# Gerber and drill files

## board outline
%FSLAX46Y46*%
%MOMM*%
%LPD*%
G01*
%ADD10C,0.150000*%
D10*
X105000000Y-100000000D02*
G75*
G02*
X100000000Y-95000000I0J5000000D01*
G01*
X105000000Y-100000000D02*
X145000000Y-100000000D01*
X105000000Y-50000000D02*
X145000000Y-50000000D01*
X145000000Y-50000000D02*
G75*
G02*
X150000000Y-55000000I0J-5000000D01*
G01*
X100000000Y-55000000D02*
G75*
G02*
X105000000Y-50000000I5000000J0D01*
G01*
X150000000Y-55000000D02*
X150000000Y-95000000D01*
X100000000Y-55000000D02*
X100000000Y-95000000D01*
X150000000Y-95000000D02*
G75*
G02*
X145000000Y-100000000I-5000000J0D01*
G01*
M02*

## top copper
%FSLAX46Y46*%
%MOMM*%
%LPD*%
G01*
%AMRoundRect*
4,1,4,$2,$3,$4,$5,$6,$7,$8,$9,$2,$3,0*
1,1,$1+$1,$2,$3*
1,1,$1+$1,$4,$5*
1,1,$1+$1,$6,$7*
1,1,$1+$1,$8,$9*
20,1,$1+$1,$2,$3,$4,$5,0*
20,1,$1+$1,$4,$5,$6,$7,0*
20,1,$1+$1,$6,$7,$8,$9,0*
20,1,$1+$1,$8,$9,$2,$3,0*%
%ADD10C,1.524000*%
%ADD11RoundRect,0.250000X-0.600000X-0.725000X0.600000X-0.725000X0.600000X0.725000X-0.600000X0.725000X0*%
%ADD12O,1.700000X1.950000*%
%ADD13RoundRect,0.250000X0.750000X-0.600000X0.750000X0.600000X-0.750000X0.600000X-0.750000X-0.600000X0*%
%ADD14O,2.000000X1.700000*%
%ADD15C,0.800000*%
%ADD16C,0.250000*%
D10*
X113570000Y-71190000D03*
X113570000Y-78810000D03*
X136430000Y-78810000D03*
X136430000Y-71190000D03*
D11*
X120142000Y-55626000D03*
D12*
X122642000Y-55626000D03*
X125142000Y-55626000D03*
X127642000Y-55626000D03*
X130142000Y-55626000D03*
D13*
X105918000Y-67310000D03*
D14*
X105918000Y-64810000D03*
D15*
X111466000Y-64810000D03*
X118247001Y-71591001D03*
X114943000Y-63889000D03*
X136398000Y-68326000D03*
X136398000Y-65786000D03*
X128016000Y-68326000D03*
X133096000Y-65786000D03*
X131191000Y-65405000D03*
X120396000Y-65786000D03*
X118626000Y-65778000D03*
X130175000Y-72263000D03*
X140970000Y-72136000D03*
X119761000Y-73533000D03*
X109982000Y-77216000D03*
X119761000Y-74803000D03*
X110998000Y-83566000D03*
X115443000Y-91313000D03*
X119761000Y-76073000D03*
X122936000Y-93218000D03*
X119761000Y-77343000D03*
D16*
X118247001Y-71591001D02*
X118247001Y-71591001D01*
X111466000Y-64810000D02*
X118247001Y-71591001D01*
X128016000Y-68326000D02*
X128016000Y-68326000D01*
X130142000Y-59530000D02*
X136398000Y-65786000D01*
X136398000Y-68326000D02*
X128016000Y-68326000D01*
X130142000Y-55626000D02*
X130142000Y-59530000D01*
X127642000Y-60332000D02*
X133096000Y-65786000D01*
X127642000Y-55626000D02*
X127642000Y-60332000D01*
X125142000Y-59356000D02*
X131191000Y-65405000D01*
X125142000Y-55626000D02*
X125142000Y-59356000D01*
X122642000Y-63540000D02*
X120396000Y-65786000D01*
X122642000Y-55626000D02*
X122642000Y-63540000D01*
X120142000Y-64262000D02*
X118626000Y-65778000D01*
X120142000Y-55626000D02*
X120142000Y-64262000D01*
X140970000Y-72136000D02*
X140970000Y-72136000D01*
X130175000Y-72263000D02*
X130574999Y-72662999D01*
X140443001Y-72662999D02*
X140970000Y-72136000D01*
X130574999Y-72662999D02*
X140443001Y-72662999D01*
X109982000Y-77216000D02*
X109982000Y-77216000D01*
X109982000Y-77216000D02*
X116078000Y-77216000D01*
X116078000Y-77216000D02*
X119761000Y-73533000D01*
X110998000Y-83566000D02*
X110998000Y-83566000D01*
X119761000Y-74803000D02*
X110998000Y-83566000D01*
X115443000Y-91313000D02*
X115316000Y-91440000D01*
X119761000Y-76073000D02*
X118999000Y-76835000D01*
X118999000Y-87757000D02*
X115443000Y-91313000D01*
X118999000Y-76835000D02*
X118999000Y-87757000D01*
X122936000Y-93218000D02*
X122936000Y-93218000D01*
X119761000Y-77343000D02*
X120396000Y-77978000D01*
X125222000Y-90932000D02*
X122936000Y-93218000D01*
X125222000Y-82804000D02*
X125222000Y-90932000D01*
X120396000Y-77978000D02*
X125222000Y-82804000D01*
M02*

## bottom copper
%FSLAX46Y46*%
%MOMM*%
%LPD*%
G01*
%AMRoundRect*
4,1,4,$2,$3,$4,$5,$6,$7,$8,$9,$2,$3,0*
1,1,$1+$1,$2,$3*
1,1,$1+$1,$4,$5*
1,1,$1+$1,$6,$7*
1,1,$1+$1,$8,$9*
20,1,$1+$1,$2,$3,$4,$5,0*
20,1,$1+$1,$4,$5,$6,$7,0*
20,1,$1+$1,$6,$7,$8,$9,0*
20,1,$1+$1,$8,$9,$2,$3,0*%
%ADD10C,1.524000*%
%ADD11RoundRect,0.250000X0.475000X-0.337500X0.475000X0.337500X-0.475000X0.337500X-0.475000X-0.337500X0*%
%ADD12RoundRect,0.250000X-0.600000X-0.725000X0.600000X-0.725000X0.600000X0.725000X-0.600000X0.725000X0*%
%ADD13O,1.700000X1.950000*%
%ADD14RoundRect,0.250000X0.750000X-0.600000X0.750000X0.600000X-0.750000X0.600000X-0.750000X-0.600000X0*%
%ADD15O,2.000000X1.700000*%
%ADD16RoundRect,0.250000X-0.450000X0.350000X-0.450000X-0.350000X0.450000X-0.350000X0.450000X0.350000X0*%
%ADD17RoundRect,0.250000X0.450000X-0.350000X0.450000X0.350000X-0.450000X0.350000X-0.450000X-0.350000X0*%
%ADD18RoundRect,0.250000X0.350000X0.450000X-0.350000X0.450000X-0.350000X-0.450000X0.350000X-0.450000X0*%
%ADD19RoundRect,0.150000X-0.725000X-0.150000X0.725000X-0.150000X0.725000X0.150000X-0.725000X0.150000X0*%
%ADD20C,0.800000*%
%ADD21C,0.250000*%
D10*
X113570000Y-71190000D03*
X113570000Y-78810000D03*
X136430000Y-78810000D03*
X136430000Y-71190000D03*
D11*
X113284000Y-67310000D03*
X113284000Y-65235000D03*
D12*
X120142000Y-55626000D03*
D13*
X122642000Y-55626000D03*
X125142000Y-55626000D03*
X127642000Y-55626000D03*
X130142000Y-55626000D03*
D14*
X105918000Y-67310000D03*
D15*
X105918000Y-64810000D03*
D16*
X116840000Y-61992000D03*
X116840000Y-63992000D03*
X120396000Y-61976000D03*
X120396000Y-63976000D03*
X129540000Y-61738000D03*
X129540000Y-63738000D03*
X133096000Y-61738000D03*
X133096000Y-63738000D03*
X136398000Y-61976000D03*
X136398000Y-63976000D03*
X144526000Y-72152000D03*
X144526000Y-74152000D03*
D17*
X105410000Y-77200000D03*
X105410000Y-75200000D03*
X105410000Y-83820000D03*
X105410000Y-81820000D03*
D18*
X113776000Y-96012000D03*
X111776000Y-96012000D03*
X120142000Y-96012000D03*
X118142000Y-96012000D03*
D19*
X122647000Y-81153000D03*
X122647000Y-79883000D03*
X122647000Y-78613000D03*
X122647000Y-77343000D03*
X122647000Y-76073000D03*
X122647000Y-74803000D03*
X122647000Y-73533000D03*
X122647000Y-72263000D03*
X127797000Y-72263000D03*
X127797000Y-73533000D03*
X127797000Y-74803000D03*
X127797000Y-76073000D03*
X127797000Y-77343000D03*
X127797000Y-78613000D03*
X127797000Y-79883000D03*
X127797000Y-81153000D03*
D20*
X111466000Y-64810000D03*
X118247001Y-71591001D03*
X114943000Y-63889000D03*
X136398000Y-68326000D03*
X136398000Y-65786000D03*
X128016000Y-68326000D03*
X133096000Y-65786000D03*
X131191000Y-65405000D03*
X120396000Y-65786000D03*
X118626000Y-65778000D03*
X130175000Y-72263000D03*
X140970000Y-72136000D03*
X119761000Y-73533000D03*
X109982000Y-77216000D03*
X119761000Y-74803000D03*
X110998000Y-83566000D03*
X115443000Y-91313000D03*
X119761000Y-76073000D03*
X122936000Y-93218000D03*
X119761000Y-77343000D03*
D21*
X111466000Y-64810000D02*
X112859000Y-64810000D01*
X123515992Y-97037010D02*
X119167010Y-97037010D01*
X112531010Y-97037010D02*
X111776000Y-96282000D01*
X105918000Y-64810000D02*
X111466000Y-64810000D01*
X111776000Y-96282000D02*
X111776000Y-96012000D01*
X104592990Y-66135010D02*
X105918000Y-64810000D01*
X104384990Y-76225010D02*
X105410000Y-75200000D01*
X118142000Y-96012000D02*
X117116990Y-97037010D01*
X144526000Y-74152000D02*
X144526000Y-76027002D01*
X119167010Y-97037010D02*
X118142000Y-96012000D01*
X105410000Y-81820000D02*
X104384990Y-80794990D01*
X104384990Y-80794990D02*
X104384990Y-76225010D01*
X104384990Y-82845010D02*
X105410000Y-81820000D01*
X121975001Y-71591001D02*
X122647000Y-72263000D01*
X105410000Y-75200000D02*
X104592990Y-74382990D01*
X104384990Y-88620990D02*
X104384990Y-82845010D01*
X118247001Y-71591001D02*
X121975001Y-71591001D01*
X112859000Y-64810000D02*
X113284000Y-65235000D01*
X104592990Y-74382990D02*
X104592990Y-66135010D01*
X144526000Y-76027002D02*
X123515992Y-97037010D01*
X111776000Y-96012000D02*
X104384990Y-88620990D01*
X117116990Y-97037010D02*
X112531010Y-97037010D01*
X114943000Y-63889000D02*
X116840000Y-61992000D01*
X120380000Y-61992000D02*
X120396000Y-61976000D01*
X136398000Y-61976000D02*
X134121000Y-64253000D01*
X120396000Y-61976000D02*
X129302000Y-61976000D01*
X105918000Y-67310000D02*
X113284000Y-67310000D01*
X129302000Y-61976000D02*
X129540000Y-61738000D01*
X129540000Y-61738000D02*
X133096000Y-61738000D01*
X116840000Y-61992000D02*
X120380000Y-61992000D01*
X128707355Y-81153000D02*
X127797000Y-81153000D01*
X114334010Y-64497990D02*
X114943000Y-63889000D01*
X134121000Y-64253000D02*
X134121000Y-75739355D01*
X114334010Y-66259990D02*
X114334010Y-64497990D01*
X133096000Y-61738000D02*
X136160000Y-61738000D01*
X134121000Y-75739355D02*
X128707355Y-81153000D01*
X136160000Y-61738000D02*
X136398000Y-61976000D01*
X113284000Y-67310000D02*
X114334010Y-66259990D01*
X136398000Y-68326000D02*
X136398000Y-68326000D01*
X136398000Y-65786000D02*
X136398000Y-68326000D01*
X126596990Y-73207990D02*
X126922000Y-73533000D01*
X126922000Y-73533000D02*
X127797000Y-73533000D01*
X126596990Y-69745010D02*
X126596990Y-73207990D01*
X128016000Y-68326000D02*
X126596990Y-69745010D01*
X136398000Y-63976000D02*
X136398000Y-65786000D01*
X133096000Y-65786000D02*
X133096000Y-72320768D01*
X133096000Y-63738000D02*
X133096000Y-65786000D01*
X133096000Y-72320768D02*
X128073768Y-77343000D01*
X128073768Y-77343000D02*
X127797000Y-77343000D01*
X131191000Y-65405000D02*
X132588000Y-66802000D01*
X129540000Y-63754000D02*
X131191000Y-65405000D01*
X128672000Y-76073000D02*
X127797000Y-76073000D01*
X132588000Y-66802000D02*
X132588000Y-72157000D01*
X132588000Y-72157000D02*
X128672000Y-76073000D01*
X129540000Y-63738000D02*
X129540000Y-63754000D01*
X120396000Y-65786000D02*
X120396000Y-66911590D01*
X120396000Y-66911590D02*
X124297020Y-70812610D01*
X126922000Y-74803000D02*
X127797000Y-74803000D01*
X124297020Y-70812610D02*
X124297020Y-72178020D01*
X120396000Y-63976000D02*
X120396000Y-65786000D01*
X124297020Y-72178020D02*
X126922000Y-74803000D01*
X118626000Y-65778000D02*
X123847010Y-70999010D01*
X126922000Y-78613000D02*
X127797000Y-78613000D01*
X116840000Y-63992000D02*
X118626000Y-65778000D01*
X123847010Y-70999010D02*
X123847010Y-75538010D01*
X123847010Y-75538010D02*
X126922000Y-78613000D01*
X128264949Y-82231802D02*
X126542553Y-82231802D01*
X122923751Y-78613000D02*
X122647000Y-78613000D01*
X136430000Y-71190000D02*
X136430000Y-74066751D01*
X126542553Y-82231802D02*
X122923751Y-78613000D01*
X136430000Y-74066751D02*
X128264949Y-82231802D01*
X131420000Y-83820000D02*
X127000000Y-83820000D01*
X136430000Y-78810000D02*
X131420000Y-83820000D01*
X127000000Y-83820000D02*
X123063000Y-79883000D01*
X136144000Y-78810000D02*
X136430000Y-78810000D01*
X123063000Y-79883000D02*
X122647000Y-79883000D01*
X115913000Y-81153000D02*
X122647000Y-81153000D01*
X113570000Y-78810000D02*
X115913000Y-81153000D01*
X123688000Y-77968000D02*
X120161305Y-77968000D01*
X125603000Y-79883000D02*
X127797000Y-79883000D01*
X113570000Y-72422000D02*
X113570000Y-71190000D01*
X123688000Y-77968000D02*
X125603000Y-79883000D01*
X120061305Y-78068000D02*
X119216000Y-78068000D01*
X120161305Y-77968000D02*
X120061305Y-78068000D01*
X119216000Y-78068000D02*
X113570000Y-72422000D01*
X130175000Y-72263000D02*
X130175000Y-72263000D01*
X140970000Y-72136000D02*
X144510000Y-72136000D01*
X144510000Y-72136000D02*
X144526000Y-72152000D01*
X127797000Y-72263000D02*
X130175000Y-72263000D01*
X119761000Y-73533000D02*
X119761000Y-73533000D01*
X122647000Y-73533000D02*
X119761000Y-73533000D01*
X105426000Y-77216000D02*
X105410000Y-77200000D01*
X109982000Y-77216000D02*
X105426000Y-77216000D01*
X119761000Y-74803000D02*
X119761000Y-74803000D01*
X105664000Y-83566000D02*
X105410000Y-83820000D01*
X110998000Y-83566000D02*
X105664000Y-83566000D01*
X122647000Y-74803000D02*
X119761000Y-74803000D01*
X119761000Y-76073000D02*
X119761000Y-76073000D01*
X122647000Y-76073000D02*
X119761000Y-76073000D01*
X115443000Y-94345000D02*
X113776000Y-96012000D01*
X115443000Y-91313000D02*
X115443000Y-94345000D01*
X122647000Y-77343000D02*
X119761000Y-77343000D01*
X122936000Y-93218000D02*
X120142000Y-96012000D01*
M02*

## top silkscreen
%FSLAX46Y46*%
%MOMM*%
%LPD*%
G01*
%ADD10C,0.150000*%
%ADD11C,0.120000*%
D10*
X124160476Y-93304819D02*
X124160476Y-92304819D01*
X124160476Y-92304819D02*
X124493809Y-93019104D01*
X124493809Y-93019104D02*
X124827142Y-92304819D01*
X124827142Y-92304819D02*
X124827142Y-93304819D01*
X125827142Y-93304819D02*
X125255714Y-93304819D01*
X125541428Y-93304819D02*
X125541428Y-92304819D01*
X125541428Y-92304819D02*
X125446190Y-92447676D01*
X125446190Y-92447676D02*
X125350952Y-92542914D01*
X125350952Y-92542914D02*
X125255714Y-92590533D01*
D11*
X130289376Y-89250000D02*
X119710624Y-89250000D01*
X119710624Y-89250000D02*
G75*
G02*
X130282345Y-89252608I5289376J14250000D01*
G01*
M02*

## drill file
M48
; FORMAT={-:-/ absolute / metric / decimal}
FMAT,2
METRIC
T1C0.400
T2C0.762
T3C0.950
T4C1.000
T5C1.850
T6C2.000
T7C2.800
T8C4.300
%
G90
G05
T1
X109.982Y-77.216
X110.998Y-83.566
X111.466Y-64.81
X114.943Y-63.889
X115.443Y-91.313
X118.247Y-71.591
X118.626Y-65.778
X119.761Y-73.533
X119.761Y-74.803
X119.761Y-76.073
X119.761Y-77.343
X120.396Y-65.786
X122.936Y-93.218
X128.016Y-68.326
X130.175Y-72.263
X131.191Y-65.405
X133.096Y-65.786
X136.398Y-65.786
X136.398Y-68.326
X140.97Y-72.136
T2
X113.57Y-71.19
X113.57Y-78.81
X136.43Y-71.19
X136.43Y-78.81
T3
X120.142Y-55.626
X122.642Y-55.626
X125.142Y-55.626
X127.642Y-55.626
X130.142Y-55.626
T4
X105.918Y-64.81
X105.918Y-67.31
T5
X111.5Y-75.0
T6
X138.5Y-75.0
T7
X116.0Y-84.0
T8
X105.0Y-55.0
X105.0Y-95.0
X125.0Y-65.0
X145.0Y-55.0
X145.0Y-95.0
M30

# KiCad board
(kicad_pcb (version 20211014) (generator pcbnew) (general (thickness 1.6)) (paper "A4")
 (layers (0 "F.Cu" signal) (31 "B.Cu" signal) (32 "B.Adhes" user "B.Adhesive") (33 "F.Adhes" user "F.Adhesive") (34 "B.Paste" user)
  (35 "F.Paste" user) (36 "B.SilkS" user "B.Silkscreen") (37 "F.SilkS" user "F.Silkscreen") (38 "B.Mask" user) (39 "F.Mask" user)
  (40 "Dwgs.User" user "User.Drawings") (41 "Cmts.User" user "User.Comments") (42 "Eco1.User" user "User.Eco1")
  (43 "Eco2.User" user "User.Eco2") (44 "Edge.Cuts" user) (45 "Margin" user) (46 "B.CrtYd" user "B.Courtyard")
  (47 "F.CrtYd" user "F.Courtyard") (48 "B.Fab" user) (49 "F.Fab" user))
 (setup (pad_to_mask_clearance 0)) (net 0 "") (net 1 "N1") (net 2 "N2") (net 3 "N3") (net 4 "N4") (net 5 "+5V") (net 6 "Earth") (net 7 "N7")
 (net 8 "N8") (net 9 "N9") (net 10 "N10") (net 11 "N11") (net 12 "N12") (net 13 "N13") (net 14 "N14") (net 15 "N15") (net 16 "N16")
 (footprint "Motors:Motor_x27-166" (layer "F.Cu") (at 125 75)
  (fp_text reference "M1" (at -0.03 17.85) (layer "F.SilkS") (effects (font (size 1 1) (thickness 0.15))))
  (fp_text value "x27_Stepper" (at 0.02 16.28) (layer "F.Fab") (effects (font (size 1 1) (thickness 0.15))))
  (fp_line (start 5.289376 14.25) (end -5.289376 14.25) (layer "F.SilkS") (width 0.12))
  (fp_arc (start -5.289376 14.25) (mid 0.00375 -15.199999) (end 5.282345 14.252608) (layer "F.SilkS") (width 0.12))
  (pad "" np_thru_hole circle (at -13.5 0) (size 1.85 1.85) (drill 1.85) (layers *.Cu *.Mask))
  (pad "" np_thru_hole circle (at 0 -10) (size 4.3 4.3) (drill 4.3) (layers *.Cu *.Mask))
  (pad "" np_thru_hole circle (at -9 9) (size 2.8 2.8) (drill 2.8) (layers *.Cu *.Mask))
  (pad "" np_thru_hole circle (at 13.5 0) (size 2 2) (drill 2) (layers *.Cu *.Mask))
  (pad "1" thru_hole circle (at -11.43 -3.81) (size 1.524 1.524) (drill 0.762) (layers *.Cu *.Mask) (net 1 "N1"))
  (pad "2" thru_hole circle (at -11.43 3.81) (size 1.524 1.524) (drill 0.762) (layers *.Cu *.Mask) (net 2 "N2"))
  (pad "3" thru_hole circle (at 11.43 3.81) (size 1.524 1.524) (drill 0.762) (layers *.Cu *.Mask) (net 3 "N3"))
  (pad "4" thru_hole circle (at 11.43 -3.81) (size 1.524 1.524) (drill 0.762) (layers *.Cu *.Mask) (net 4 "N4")))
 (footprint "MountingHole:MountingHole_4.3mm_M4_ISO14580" (layer "F.Cu") (at 105 55)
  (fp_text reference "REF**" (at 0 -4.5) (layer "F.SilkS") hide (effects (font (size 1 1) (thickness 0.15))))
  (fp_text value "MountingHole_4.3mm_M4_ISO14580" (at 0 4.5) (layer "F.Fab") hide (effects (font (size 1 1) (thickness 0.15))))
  (pad "" np_thru_hole circle locked (at 0 0) (size 4.3 4.3) (drill 4.3) (layers *.Cu *.Mask)))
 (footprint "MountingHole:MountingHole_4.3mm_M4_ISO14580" (layer "F.Cu") (at 145 55)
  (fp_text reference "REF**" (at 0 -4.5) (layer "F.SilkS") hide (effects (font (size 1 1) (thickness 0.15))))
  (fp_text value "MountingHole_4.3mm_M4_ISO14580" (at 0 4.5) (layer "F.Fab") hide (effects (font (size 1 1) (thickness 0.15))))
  (pad "" np_thru_hole circle locked (at 0 0) (size 4.3 4.3) (drill 4.3) (layers *.Cu *.Mask)))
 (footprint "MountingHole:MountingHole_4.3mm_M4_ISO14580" (layer "F.Cu") (at 105 95)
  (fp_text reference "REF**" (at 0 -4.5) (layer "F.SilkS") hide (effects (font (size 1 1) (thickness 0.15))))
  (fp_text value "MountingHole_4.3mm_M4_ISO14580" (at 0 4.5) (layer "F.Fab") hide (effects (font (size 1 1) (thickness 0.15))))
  (pad "" np_thru_hole circle locked (at 0 0) (size 4.3 4.3) (drill 4.3) (layers *.Cu *.Mask)))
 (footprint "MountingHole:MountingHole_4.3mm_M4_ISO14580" (layer "F.Cu") (at 145 95)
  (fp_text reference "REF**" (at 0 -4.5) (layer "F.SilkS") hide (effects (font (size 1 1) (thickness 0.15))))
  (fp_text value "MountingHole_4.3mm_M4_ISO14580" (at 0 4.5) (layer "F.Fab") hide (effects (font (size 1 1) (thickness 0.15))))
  (pad "" np_thru_hole circle locked (at 0 0) (size 4.3 4.3) (drill 4.3) (layers *.Cu *.Mask)))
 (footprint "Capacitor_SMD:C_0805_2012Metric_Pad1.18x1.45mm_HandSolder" (layer "B.Cu") (at 113.284 66.2725 90)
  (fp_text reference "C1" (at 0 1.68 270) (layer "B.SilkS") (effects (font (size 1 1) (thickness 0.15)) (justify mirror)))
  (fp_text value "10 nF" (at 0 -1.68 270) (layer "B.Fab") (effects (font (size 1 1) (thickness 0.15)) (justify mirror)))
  (pad "1" smd roundrect locked (at -1.0375 0 90) (size 1.175 1.45) (layers "B.Cu" "B.Paste" "B.Mask") (roundrect_rratio 0.2127659574)
   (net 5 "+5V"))
  (pad "2" smd roundrect locked (at 1.0375 0 90) (size 1.175 1.45) (layers "B.Cu" "B.Paste" "B.Mask") (roundrect_rratio 0.2127659574)
   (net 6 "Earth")))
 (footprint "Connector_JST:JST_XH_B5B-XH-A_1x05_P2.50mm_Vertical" (layer "B.Cu") (at 120.142 55.626)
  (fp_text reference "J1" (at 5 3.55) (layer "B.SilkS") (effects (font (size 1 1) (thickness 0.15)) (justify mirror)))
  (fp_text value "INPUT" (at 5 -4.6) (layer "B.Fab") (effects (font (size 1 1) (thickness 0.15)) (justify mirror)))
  (pad "1" thru_hole roundrect locked (at 0 0) (size 1.7 1.95) (drill 0.95) (layers *.Cu *.Mask) (roundrect_rratio 0.1470588235)
   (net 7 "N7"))
  (pad "2" thru_hole oval locked (at 2.5 0) (size 1.7 1.95) (drill 0.95) (layers *.Cu *.Mask) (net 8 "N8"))
  (pad "3" thru_hole oval locked (at 5 0) (size 1.7 1.95) (drill 0.95) (layers *.Cu *.Mask) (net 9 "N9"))
  (pad "4" thru_hole oval locked (at 7.5 0) (size 1.7 1.95) (drill 0.95) (layers *.Cu *.Mask) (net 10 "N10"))
  (pad "5" thru_hole oval locked (at 10 0) (size 1.7 1.95) (drill 0.95) (layers *.Cu *.Mask) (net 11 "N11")))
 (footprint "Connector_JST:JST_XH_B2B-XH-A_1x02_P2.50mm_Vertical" (layer "B.Cu") (at 105.918 67.31 90)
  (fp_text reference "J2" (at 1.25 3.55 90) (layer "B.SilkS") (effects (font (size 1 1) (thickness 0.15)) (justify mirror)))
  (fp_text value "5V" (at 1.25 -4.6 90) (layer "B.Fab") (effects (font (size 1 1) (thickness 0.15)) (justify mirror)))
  (pad "1" thru_hole roundrect locked (at 0 0 90) (size 1.7 2) (drill 1) (layers *.Cu *.Mask) (roundrect_rratio 0.1470588235) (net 5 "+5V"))
  (pad "2" thru_hole oval locked (at 2.5 0 90) (size 1.7 2) (drill 1) (layers *.Cu *.Mask) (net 6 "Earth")))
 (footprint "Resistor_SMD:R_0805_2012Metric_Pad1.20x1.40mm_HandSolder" (layer "B.Cu") (at 116.84 62.992 -90)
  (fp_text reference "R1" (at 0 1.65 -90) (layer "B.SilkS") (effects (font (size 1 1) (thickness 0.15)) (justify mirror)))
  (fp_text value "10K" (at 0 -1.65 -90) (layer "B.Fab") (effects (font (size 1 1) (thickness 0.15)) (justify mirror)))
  (pad "1" smd roundrect locked (at -1 0 270) (size 1.2 1.4) (layers "B.Cu" "B.Paste" "B.Mask") (roundrect_rratio 0.2083333333)
   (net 5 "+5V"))
  (pad "2" smd roundrect locked (at 1 0 270) (size 1.2 1.4) (layers "B.Cu" "B.Paste" "B.Mask") (roundrect_rratio 0.2083333333) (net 7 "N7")))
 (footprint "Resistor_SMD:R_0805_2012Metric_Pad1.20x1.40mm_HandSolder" (layer "B.Cu") (at 120.396 62.976 -90)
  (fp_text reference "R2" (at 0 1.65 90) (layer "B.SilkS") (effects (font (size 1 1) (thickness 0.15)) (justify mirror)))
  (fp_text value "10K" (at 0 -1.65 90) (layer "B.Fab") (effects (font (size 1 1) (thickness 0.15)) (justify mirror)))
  (pad "1" smd roundrect locked (at -1 0 270) (size 1.2 1.4) (layers "B.Cu" "B.Paste" "B.Mask") (roundrect_rratio 0.2083333333)
   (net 5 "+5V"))
  (pad "2" smd roundrect locked (at 1 0 270) (size 1.2 1.4) (layers "B.Cu" "B.Paste" "B.Mask") (roundrect_rratio 0.2083333333) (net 8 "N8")))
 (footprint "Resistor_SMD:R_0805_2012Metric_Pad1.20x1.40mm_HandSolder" (layer "B.Cu") (at 129.54 62.738 -90)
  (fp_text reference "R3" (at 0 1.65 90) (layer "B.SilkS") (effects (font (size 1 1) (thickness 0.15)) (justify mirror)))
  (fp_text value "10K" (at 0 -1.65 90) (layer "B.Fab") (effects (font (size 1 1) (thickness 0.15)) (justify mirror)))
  (pad "1" smd roundrect locked (at -1 0 270) (size 1.2 1.4) (layers "B.Cu" "B.Paste" "B.Mask") (roundrect_rratio 0.2083333333)
   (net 5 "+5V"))
  (pad "2" smd roundrect locked (at 1 0 270) (size 1.2 1.4) (layers "B.Cu" "B.Paste" "B.Mask") (roundrect_rratio 0.2083333333) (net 9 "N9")))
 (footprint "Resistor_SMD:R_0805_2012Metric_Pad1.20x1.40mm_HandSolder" (layer "B.Cu") (at 133.096 62.738 -90)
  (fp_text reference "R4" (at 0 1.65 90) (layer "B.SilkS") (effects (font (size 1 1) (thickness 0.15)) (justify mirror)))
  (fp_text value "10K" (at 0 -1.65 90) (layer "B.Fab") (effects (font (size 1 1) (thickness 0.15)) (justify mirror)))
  (pad "1" smd roundrect locked (at -1 0 270) (size 1.2 1.4) (layers "B.Cu" "B.Paste" "B.Mask") (roundrect_rratio 0.2083333333)
   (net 5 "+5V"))
  (pad "2" smd roundrect locked (at 1 0 270) (size 1.2 1.4) (layers "B.Cu" "B.Paste" "B.Mask") (roundrect_rratio 0.2083333333)
   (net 10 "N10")))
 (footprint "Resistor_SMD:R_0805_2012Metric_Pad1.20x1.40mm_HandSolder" (layer "B.Cu") (at 136.398 62.976 -90)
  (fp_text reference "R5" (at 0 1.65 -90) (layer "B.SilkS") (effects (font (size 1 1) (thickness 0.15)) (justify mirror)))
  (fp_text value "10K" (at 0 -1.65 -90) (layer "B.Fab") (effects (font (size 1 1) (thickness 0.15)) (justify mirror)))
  (pad "1" smd roundrect locked (at -1 0 270) (size 1.2 1.4) (layers "B.Cu" "B.Paste" "B.Mask") (roundrect_rratio 0.2083333333)
   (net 5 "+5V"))
  (pad "2" smd roundrect locked (at 1 0 270) (size 1.2 1.4) (layers "B.Cu" "B.Paste" "B.Mask") (roundrect_rratio 0.2083333333)
   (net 11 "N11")))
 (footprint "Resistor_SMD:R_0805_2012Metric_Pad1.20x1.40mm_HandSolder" (layer "B.Cu") (at 144.526 73.152 -90)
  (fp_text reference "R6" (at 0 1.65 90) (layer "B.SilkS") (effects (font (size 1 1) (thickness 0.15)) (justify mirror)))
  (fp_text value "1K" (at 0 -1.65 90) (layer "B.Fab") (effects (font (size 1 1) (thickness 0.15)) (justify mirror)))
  (pad "1" smd roundrect locked (at -1 0 270) (size 1.2 1.4) (layers "B.Cu" "B.Paste" "B.Mask") (roundrect_rratio 0.2083333333)
   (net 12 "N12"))
  (pad "2" smd roundrect locked (at 1 0 270) (size 1.2 1.4) (layers "B.Cu" "B.Paste" "B.Mask") (roundrect_rratio 0.2083333333)
   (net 6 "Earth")))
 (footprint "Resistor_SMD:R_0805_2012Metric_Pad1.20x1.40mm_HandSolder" (layer "B.Cu") (at 105.41 76.2 90)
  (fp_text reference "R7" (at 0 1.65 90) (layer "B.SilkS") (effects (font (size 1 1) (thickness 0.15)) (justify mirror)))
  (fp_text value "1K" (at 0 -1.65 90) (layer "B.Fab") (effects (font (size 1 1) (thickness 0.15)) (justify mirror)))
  (pad "1" smd roundrect locked (at -1 0 90) (size 1.2 1.4) (layers "B.Cu" "B.Paste" "B.Mask") (roundrect_rratio 0.2083333333)
   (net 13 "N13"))
  (pad "2" smd roundrect locked (at 1 0 90) (size 1.2 1.4) (layers "B.Cu" "B.Paste" "B.Mask") (roundrect_rratio 0.2083333333)
   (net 6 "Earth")))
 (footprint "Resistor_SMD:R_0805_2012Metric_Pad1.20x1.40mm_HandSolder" (layer "B.Cu") (at 105.41 82.82 90)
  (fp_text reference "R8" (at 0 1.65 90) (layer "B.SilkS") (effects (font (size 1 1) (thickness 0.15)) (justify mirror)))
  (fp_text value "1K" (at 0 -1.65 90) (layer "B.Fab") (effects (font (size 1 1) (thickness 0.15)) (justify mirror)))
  (pad "1" smd roundrect locked (at -1 0 90) (size 1.2 1.4) (layers "B.Cu" "B.Paste" "B.Mask") (roundrect_rratio 0.2083333333)
   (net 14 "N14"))
  (pad "2" smd roundrect locked (at 1 0 90) (size 1.2 1.4) (layers "B.Cu" "B.Paste" "B.Mask") (roundrect_rratio 0.2083333333)
   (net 6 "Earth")))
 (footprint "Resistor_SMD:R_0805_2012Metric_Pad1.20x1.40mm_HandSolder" (layer "B.Cu") (at 112.776 96.012 180)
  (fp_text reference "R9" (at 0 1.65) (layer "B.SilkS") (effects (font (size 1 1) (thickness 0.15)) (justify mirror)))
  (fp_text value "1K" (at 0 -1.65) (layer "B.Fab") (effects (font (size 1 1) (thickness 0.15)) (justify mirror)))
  (pad "1" smd roundrect locked (at -1 0 180) (size 1.2 1.4) (layers "B.Cu" "B.Paste" "B.Mask") (roundrect_rratio 0.2083333333)
   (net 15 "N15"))
  (pad "2" smd roundrect locked (at 1 0 180) (size 1.2 1.4) (layers "B.Cu" "B.Paste" "B.Mask") (roundrect_rratio 0.2083333333)
   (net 6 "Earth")))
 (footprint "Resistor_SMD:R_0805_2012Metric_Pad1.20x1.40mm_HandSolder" (layer "B.Cu") (at 119.142 96.012 180)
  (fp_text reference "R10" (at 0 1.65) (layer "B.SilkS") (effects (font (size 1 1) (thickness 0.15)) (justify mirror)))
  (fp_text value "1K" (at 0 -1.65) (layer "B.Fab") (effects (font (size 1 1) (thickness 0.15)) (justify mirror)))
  (pad "1" smd roundrect locked (at -1 0 180) (size 1.2 1.4) (layers "B.Cu" "B.Paste" "B.Mask") (roundrect_rratio 0.2083333333)
   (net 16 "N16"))
  (pad "2" smd roundrect locked (at 1 0 180) (size 1.2 1.4) (layers "B.Cu" "B.Paste" "B.Mask") (roundrect_rratio 0.2083333333)
   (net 6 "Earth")))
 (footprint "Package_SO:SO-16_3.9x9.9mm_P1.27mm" (layer "B.Cu") (at 125.222 76.708)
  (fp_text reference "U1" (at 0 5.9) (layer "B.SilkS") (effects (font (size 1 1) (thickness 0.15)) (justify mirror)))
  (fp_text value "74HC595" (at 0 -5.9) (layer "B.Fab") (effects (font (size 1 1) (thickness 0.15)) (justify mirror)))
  (pad "1" smd roundrect locked (at -2.575 4.445) (size 1.75 0.6) (layers "B.Cu" "B.Paste" "B.Mask") (roundrect_rratio 0.25) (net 2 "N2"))
  (pad "2" smd roundrect locked (at -2.575 3.175) (size 1.75 0.6) (layers "B.Cu" "B.Paste" "B.Mask") (roundrect_rratio 0.25) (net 3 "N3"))
  (pad "3" smd roundrect locked (at -2.575 1.905) (size 1.75 0.6) (layers "B.Cu" "B.Paste" "B.Mask") (roundrect_rratio 0.25) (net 4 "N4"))
  (pad "4" smd roundrect locked (at -2.575 0.635) (size 1.75 0.6) (layers "B.Cu" "B.Paste" "B.Mask") (roundrect_rratio 0.25) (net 16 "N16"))
  (pad "5" smd roundrect locked (at -2.575 -0.635) (size 1.75 0.6) (layers "B.Cu" "B.Paste" "B.Mask") (roundrect_rratio 0.25) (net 15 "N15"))
  (pad "6" smd roundrect locked (at -2.575 -1.905) (size 1.75 0.6) (layers "B.Cu" "B.Paste" "B.Mask") (roundrect_rratio 0.25) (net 14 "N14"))
  (pad "7" smd roundrect locked (at -2.575 -3.175) (size 1.75 0.6) (layers "B.Cu" "B.Paste" "B.Mask") (roundrect_rratio 0.25) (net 13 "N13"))
  (pad "8" smd roundrect locked (at -2.575 -4.445) (size 1.75 0.6) (layers "B.Cu" "B.Paste" "B.Mask") (roundrect_rratio 0.25)
   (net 6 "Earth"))
  (pad "9" smd roundrect locked (at 2.575 -4.445) (size 1.75 0.6) (layers "B.Cu" "B.Paste" "B.Mask") (roundrect_rratio 0.25) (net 12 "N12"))
  (pad "10" smd roundrect locked (at 2.575 -3.175) (size 1.75 0.6) (layers "B.Cu" "B.Paste" "B.Mask") (roundrect_rratio 0.25) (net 11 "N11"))
  (pad "11" smd roundrect locked (at 2.575 -1.905) (size 1.75 0.6) (layers "B.Cu" "B.Paste" "B.Mask") (roundrect_rratio 0.25) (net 8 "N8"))
  (pad "12" smd roundrect locked (at 2.575 -0.635) (size 1.75 0.6) (layers "B.Cu" "B.Paste" "B.Mask") (roundrect_rratio 0.25) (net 9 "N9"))
  (pad "13" smd roundrect locked (at 2.575 0.635) (size 1.75 0.6) (layers "B.Cu" "B.Paste" "B.Mask") (roundrect_rratio 0.25) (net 10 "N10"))
  (pad "14" smd roundrect locked (at 2.575 1.905) (size 1.75 0.6) (layers "B.Cu" "B.Paste" "B.Mask") (roundrect_rratio 0.25) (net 7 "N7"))
  (pad "15" smd roundrect locked (at 2.575 3.175) (size 1.75 0.6) (layers "B.Cu" "B.Paste" "B.Mask") (roundrect_rratio 0.25) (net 1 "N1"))
  (pad "16" smd roundrect locked (at 2.575 4.445) (size 1.75 0.6) (layers "B.Cu" "B.Paste" "B.Mask") (roundrect_rratio 0.25) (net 5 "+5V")))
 (gr_arc (start 105 100) (mid 101.464466 98.535534) (end 100 95) (layer "Edge.Cuts") (width 0.15))
 (gr_line (start 105 100) (end 145 100) (layer "Edge.Cuts") (width 0.15))
 (gr_line (start 105 50) (end 145 50) (layer "Edge.Cuts") (width 0.15))
 (gr_arc (start 145 50) (mid 148.535534 51.464466) (end 150 55) (layer "Edge.Cuts") (width 0.15))
 (gr_arc (start 100 55) (mid 101.464466 51.464466) (end 105 50) (layer "Edge.Cuts") (width 0.15))
 (gr_line (start 150 55) (end 150 95) (layer "Edge.Cuts") (width 0.15))
 (gr_line (start 100 55) (end 100 95) (layer "Edge.Cuts") (width 0.15))
 (gr_arc (start 150 95) (mid 148.535534 98.535534) (end 145 100) (layer "Edge.Cuts") (width 0.15))
 (segment (start 118.247001 71.591001) (end 118.247001 71.591001) (width 0.25) (layer "F.Cu") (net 6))
 (segment (start 111.466 64.81) (end 118.247001 71.591001) (width 0.25) (layer "F.Cu") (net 6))
 (via (at 111.466 64.81) (size 0.8) (drill 0.4) (layers "F.Cu" "B.Cu") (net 6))
 (via (at 118.247001 71.591001) (size 0.8) (drill 0.4) (layers "F.Cu" "B.Cu") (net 6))
 (segment (start 111.466 64.81) (end 112.859 64.81) (width 0.25) (layer "B.Cu") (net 6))
 (segment (start 123.515992 97.03701) (end 119.16701 97.03701) (width 0.25) (layer "B.Cu") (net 6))
 (segment (start 112.53101 97.03701) (end 111.776 96.282) (width 0.25) (layer "B.Cu") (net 6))
 (segment (start 105.918 64.81) (end 111.466 64.81) (width 0.25) (layer "B.Cu") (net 6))
 (segment (start 111.776 96.282) (end 111.776 96.012) (width 0.25) (layer "B.Cu") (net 6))
 (segment (start 104.59299 66.13501) (end 105.918 64.81) (width 0.25) (layer "B.Cu") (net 6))
 (segment (start 104.38499 76.22501) (end 105.41 75.2) (width 0.25) (layer "B.Cu") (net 6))
 (segment (start 118.142 96.012) (end 117.11699 97.03701) (width 0.25) (layer "B.Cu") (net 6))
 (segment (start 144.526 74.152) (end 144.526 76.027002) (width 0.25) (layer "B.Cu") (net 6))
 (segment (start 119.16701 97.03701) (end 118.142 96.012) (width 0.25) (layer "B.Cu") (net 6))
 (segment (start 105.41 81.82) (end 104.38499 80.79499) (width 0.25) (layer "B.Cu") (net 6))
 (segment (start 104.38499 80.79499) (end 104.38499 76.22501) (width 0.25) (layer "B.Cu") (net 6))
 (segment (start 104.38499 82.84501) (end 105.41 81.82) (width 0.25) (layer "B.Cu") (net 6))
 (segment (start 121.975001 71.591001) (end 122.647 72.263) (width 0.25) (layer "B.Cu") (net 6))
 (segment (start 105.41 75.2) (end 104.59299 74.38299) (width 0.25) (layer "B.Cu") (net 6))
 (segment (start 104.38499 88.62099) (end 104.38499 82.84501) (width 0.25) (layer "B.Cu") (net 6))
 (segment (start 118.247001 71.591001) (end 121.975001 71.591001) (width 0.25) (layer "B.Cu") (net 6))
 (segment (start 112.859 64.81) (end 113.284 65.235) (width 0.25) (layer "B.Cu") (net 6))
 (segment (start 104.59299 74.38299) (end 104.59299 66.13501) (width 0.25) (layer "B.Cu") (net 6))
 (segment (start 144.526 76.027002) (end 123.515992 97.03701) (width 0.25) (layer "B.Cu") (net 6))
 (segment (start 111.776 96.012) (end 104.38499 88.62099) (width 0.25) (layer "B.Cu") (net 6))
 (segment (start 117.11699 97.03701) (end 112.53101 97.03701) (width 0.25) (layer "B.Cu") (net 6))
 (via (at 114.943 63.889) (size 0.8) (drill 0.4) (layers "F.Cu" "B.Cu") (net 5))
 (segment (start 114.943 63.889) (end 116.84 61.992) (width 0.25) (layer "B.Cu") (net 5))
 (segment (start 120.38 61.992) (end 120.396 61.976) (width 0.25) (layer "B.Cu") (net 5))
 (segment (start 136.398 61.976) (end 134.121 64.253) (width 0.25) (layer "B.Cu") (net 5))
 (segment (start 120.396 61.976) (end 129.302 61.976) (width 0.25) (layer "B.Cu") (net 5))
 (segment (start 105.918 67.31) (end 113.284 67.31) (width 0.25) (layer "B.Cu") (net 5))
 (segment (start 129.302 61.976) (end 129.54 61.738) (width 0.25) (layer "B.Cu") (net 5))
 (segment (start 129.54 61.738) (end 133.096 61.738) (width 0.25) (layer "B.Cu") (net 5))
 (segment (start 116.84 61.992) (end 120.38 61.992) (width 0.25) (layer "B.Cu") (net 5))
 (segment (start 128.707355 81.153) (end 127.797 81.153) (width 0.25) (layer "B.Cu") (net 5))
 (segment (start 114.33401 64.49799) (end 114.943 63.889) (width 0.25) (layer "B.Cu") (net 5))
 (segment (start 134.121 64.253) (end 134.121 75.739355) (width 0.25) (layer "B.Cu") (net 5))
 (segment (start 114.33401 66.25999) (end 114.33401 64.49799) (width 0.25) (layer "B.Cu") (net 5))
 (segment (start 133.096 61.738) (end 136.16 61.738) (width 0.25) (layer "B.Cu") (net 5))
 (segment (start 134.121 75.739355) (end 128.707355 81.153) (width 0.25) (layer "B.Cu") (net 5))
 (segment (start 136.16 61.738) (end 136.398 61.976) (width 0.25) (layer "B.Cu") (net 5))
 (segment (start 113.284 67.31) (end 114.33401 66.25999) (width 0.25) (layer "B.Cu") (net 5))
 (segment (start 128.016 68.326) (end 128.016 68.326) (width 0.25) (layer "F.Cu") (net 11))
 (segment (start 130.142 59.53) (end 136.398 65.786) (width 0.25) (layer "F.Cu") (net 11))
 (segment (start 136.398 68.326) (end 128.016 68.326) (width 0.25) (layer "F.Cu") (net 11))
 (segment (start 130.142 55.626) (end 130.142 59.53) (width 0.25) (layer "F.Cu") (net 11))
 (via (at 136.398 68.326) (size 0.8) (drill 0.4) (layers "F.Cu" "B.Cu") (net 11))
 (via (at 136.398 65.786) (size 0.8) (drill 0.4) (layers "F.Cu" "B.Cu") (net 11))
 (via (at 128.016 68.326) (size 0.8) (drill 0.4) (layers "F.Cu" "B.Cu") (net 11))
 (segment (start 136.398 68.326) (end 136.398 68.326) (width 0.25) (layer "B.Cu") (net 11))
 (segment (start 136.398 65.786) (end 136.398 68.326) (width 0.25) (layer "B.Cu") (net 11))
 (segment (start 126.59699 73.20799) (end 126.922 73.533) (width 0.25) (layer "B.Cu") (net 11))
 (segment (start 126.922 73.533) (end 127.797 73.533) (width 0.25) (layer "B.Cu") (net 11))
 (segment (start 126.59699 69.74501) (end 126.59699 73.20799) (width 0.25) (layer "B.Cu") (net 11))
 (segment (start 128.016 68.326) (end 126.59699 69.74501) (width 0.25) (layer "B.Cu") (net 11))
 (segment (start 136.398 63.976) (end 136.398 65.786) (width 0.25) (layer "B.Cu") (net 11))
 (segment (start 127.642 60.332) (end 133.096 65.786) (width 0.25) (layer "F.Cu") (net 10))
 (segment (start 127.642 55.626) (end 127.642 60.332) (width 0.25) (layer "F.Cu") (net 10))
 (via (at 133.096 65.786) (size 0.8) (drill 0.4) (layers "F.Cu" "B.Cu") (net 10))
 (segment (start 133.096 65.786) (end 133.096 72.320768) (width 0.25) (layer "B.Cu") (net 10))
 (segment (start 133.096 63.738) (end 133.096 65.786) (width 0.25) (layer "B.Cu") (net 10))
 (segment (start 133.096 72.320768) (end 128.073768 77.343) (width 0.25) (layer "B.Cu") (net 10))
 (segment (start 128.073768 77.343) (end 127.797 77.343) (width 0.25) (layer "B.Cu") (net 10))
 (segment (start 125.142 59.356) (end 131.191 65.405) (width 0.25) (layer "F.Cu") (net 9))
 (segment (start 125.142 55.626) (end 125.142 59.356) (width 0.25) (layer "F.Cu") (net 9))
 (via (at 131.191 65.405) (size 0.8) (drill 0.4) (layers "F.Cu" "B.Cu") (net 9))
 (segment (start 131.191 65.405) (end 132.588 66.802) (width 0.25) (layer "B.Cu") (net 9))
 (segment (start 129.54 63.754) (end 131.191 65.405) (width 0.25) (layer "B.Cu") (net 9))
 (segment (start 128.672 76.073) (end 127.797 76.073) (width 0.25) (layer "B.Cu") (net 9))
 (segment (start 132.588 66.802) (end 132.588 72.157) (width 0.25) (layer "B.Cu") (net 9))
 (segment (start 132.588 72.157) (end 128.672 76.073) (width 0.25) (layer "B.Cu") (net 9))
 (segment (start 129.54 63.738) (end 129.54 63.754) (width 0.25) (layer "B.Cu") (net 9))
 (segment (start 122.642 63.54) (end 120.396 65.786) (width 0.25) (layer "F.Cu") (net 8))
 (segment (start 122.642 55.626) (end 122.642 63.54) (width 0.25) (layer "F.Cu") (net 8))
 (via (at 120.396 65.786) (size 0.8) (drill 0.4) (layers "F.Cu" "B.Cu") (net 8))
 (segment (start 120.396 65.786) (end 120.396 66.91159) (width 0.25) (layer "B.Cu") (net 8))
 (segment (start 120.396 66.91159) (end 124.29702 70.81261) (width 0.25) (layer "B.Cu") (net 8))
 (segment (start 126.922 74.803) (end 127.797 74.803) (width 0.25) (layer "B.Cu") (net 8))
 (segment (start 124.29702 70.81261) (end 124.29702 72.17802) (width 0.25) (layer "B.Cu") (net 8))
 (segment (start 120.396 63.976) (end 120.396 65.786) (width 0.25) (layer "B.Cu") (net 8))
 (segment (start 124.29702 72.17802) (end 126.922 74.803) (width 0.25) (layer "B.Cu") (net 8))
 (segment (start 120.142 64.262) (end 118.626 65.778) (width 0.25) (layer "F.Cu") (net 7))
 (segment (start 120.142 55.626) (end 120.142 64.262) (width 0.25) (layer "F.Cu") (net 7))
 (via (at 118.626 65.778) (size 0.8) (drill 0.4) (layers "F.Cu" "B.Cu") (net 7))
 (segment (start 118.626 65.778) (end 123.84701 70.99901) (width 0.25) (layer "B.Cu") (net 7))
 (segment (start 126.922 78.613) (end 127.797 78.613) (width 0.25) (layer "B.Cu") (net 7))
 (segment (start 116.84 63.992) (end 118.626 65.778) (width 0.25) (layer "B.Cu") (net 7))
 (segment (start 123.84701 70.99901) (end 123.84701 75.53801) (width 0.25) (layer "B.Cu") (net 7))
 (segment (start 123.84701 75.53801) (end 126.922 78.613) (width 0.25) (layer "B.Cu") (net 7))
 (segment (start 128.264949 82.231802) (end 126.542553 82.231802) (width 0.25) (layer "B.Cu") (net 4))
 (segment (start 122.923751 78.613) (end 122.647 78.613) (width 0.25) (layer "B.Cu") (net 4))
 (segment (start 136.43 71.19) (end 136.43 74.066751) (width 0.25) (layer "B.Cu") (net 4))
 (segment (start 126.542553 82.231802) (end 122.923751 78.613) (width 0.25) (layer "B.Cu") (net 4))
 (segment (start 136.43 74.066751) (end 128.264949 82.231802) (width 0.25) (layer "B.Cu") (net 4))
 (segment (start 131.42 83.82) (end 127 83.82) (width 0.25) (layer "B.Cu") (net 3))
 (segment (start 136.43 78.81) (end 131.42 83.82) (width 0.25) (layer "B.Cu") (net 3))
 (segment (start 127 83.82) (end 123.063 79.883) (width 0.25) (layer "B.Cu") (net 3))
 (segment (start 136.144 78.81) (end 136.43 78.81) (width 0.25) (layer "B.Cu") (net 3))
 (segment (start 123.063 79.883) (end 122.647 79.883) (width 0.25) (layer "B.Cu") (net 3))
 (segment (start 115.913 81.153) (end 122.647 81.153) (width 0.25) (layer "B.Cu") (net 2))
 (segment (start 113.57 78.81) (end 115.913 81.153) (width 0.25) (layer "B.Cu") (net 2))
 (segment (start 123.688 77.968) (end 120.161305 77.968) (width 0.25) (layer "B.Cu") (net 1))
 (segment (start 125.603 79.883) (end 127.797 79.883) (width 0.25) (layer "B.Cu") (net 1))
 (segment (start 113.57 72.422) (end 113.57 71.19) (width 0.25) (layer "B.Cu") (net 1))
 (segment (start 123.688 77.968) (end 125.603 79.883) (width 0.25) (layer "B.Cu") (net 1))
 (segment (start 120.061305 78.068) (end 119.216 78.068) (width 0.25) (layer "B.Cu") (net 1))
 (segment (start 120.161305 77.968) (end 120.061305 78.068) (width 0.25) (layer "B.Cu") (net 1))
 (segment (start 119.216 78.068) (end 113.57 72.422) (width 0.25) (layer "B.Cu") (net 1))
 (segment (start 140.97 72.136) (end 140.97 72.136) (width 0.25) (layer "F.Cu") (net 12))
 (segment (start 130.175 72.263) (end 130.574999 72.662999) (width 0.25) (layer "F.Cu") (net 12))
 (segment (start 140.443001 72.662999) (end 140.97 72.136) (width 0.25) (layer "F.Cu") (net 12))
 (segment (start 130.574999 72.662999) (end 140.443001 72.662999) (width 0.25) (layer "F.Cu") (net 12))
 (via (at 130.175 72.263) (size 0.8) (drill 0.4) (layers "F.Cu" "B.Cu") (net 12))
 (via (at 140.97 72.136) (size 0.8) (drill 0.4) (layers "F.Cu" "B.Cu") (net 12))
 (segment (start 130.175 72.263) (end 130.175 72.263) (width 0.25) (layer "B.Cu") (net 12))
 (segment (start 140.97 72.136) (end 144.51 72.136) (width 0.25) (layer "B.Cu") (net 12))
 (segment (start 144.51 72.136) (end 144.526 72.152) (width 0.25) (layer "B.Cu") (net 12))
 (segment (start 127.797 72.263) (end 130.175 72.263) (width 0.25) (layer "B.Cu") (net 12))
 (segment (start 109.982 77.216) (end 109.982 77.216) (width 0.25) (layer "F.Cu") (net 13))
 (segment (start 109.982 77.216) (end 116.078 77.216) (width 0.25) (layer "F.Cu") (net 13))
 (segment (start 116.078 77.216) (end 119.761 73.533) (width 0.25) (layer "F.Cu") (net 13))
 (via (at 119.761 73.533) (size 0.8) (drill 0.4) (layers "F.Cu" "B.Cu") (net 13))
 (via (at 109.982 77.216) (size 0.8) (drill 0.4) (layers "F.Cu" "B.Cu") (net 13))
 (segment (start 119.761 73.533) (end 119.761 73.533) (width 0.25) (layer "B.Cu") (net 13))
 (segment (start 122.647 73.533) (end 119.761 73.533) (width 0.25) (layer "B.Cu") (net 13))
 (segment (start 105.426 77.216) (end 105.41 77.2) (width 0.25) (layer "B.Cu") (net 13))
 (segment (start 109.982 77.216) (end 105.426 77.216) (width 0.25) (layer "B.Cu") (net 13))
 (segment (start 110.998 83.566) (end 110.998 83.566) (width 0.25) (layer "F.Cu") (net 14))
 (segment (start 119.761 74.803) (end 110.998 83.566) (width 0.25) (layer "F.Cu") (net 14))
 (via (at 119.761 74.803) (size 0.8) (drill 0.4) (layers "F.Cu" "B.Cu") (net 14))
 (via (at 110.998 83.566) (size 0.8) (drill 0.4) (layers "F.Cu" "B.Cu") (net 14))
 (segment (start 119.761 74.803) (end 119.761 74.803) (width 0.25) (layer "B.Cu") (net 14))
 (segment (start 105.664 83.566) (end 105.41 83.82) (width 0.25) (layer "B.Cu") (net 14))
 (segment (start 110.998 83.566) (end 105.664 83.566) (width 0.25) (layer "B.Cu") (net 14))
 (segment (start 122.647 74.803) (end 119.761 74.803) (width 0.25) (layer "B.Cu") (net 14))
 (segment (start 115.443 91.313) (end 115.316 91.44) (width 0.25) (layer "F.Cu") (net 15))
 (segment (start 119.761 76.073) (end 118.999 76.835) (width 0.25) (layer "F.Cu") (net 15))
 (segment (start 118.999 87.757) (end 115.443 91.313) (width 0.25) (layer "F.Cu") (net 15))
 (segment (start 118.999 76.835) (end 118.999 87.757) (width 0.25) (layer "F.Cu") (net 15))
 (via (at 115.443 91.313) (size 0.8) (drill 0.4) (layers "F.Cu" "B.Cu") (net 15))
 (via (at 119.761 76.073) (size 0.8) (drill 0.4) (layers "F.Cu" "B.Cu") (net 15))
 (segment (start 119.761 76.073) (end 119.761 76.073) (width 0.25) (layer "B.Cu") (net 15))
 (segment (start 122.647 76.073) (end 119.761 76.073) (width 0.25) (layer "B.Cu") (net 15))
 (segment (start 115.443 94.345) (end 113.776 96.012) (width 0.25) (layer "B.Cu") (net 15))
 (segment (start 115.443 91.313) (end 115.443 94.345) (width 0.25) (layer "B.Cu") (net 15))
 (segment (start 122.936 93.218) (end 122.936 93.218) (width 0.25) (layer "F.Cu") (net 16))
 (segment (start 119.761 77.343) (end 120.396 77.978) (width 0.25) (layer "F.Cu") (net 16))
 (segment (start 125.222 90.932) (end 122.936 93.218) (width 0.25) (layer "F.Cu") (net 16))
 (segment (start 125.222 82.804) (end 125.222 90.932) (width 0.25) (layer "F.Cu") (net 16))
 (segment (start 120.396 77.978) (end 125.222 82.804) (width 0.25) (layer "F.Cu") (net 16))
 (via (at 122.936 93.218) (size 0.8) (drill 0.4) (layers "F.Cu" "B.Cu") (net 16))
 (via (at 119.761 77.343) (size 0.8) (drill 0.4) (layers "F.Cu" "B.Cu") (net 16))
 (segment (start 122.647 77.343) (end 119.761 77.343) (width 0.25) (layer "B.Cu") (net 16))
 (segment (start 122.936 93.218) (end 120.142 96.012) (width 0.25) (layer "B.Cu") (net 16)))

